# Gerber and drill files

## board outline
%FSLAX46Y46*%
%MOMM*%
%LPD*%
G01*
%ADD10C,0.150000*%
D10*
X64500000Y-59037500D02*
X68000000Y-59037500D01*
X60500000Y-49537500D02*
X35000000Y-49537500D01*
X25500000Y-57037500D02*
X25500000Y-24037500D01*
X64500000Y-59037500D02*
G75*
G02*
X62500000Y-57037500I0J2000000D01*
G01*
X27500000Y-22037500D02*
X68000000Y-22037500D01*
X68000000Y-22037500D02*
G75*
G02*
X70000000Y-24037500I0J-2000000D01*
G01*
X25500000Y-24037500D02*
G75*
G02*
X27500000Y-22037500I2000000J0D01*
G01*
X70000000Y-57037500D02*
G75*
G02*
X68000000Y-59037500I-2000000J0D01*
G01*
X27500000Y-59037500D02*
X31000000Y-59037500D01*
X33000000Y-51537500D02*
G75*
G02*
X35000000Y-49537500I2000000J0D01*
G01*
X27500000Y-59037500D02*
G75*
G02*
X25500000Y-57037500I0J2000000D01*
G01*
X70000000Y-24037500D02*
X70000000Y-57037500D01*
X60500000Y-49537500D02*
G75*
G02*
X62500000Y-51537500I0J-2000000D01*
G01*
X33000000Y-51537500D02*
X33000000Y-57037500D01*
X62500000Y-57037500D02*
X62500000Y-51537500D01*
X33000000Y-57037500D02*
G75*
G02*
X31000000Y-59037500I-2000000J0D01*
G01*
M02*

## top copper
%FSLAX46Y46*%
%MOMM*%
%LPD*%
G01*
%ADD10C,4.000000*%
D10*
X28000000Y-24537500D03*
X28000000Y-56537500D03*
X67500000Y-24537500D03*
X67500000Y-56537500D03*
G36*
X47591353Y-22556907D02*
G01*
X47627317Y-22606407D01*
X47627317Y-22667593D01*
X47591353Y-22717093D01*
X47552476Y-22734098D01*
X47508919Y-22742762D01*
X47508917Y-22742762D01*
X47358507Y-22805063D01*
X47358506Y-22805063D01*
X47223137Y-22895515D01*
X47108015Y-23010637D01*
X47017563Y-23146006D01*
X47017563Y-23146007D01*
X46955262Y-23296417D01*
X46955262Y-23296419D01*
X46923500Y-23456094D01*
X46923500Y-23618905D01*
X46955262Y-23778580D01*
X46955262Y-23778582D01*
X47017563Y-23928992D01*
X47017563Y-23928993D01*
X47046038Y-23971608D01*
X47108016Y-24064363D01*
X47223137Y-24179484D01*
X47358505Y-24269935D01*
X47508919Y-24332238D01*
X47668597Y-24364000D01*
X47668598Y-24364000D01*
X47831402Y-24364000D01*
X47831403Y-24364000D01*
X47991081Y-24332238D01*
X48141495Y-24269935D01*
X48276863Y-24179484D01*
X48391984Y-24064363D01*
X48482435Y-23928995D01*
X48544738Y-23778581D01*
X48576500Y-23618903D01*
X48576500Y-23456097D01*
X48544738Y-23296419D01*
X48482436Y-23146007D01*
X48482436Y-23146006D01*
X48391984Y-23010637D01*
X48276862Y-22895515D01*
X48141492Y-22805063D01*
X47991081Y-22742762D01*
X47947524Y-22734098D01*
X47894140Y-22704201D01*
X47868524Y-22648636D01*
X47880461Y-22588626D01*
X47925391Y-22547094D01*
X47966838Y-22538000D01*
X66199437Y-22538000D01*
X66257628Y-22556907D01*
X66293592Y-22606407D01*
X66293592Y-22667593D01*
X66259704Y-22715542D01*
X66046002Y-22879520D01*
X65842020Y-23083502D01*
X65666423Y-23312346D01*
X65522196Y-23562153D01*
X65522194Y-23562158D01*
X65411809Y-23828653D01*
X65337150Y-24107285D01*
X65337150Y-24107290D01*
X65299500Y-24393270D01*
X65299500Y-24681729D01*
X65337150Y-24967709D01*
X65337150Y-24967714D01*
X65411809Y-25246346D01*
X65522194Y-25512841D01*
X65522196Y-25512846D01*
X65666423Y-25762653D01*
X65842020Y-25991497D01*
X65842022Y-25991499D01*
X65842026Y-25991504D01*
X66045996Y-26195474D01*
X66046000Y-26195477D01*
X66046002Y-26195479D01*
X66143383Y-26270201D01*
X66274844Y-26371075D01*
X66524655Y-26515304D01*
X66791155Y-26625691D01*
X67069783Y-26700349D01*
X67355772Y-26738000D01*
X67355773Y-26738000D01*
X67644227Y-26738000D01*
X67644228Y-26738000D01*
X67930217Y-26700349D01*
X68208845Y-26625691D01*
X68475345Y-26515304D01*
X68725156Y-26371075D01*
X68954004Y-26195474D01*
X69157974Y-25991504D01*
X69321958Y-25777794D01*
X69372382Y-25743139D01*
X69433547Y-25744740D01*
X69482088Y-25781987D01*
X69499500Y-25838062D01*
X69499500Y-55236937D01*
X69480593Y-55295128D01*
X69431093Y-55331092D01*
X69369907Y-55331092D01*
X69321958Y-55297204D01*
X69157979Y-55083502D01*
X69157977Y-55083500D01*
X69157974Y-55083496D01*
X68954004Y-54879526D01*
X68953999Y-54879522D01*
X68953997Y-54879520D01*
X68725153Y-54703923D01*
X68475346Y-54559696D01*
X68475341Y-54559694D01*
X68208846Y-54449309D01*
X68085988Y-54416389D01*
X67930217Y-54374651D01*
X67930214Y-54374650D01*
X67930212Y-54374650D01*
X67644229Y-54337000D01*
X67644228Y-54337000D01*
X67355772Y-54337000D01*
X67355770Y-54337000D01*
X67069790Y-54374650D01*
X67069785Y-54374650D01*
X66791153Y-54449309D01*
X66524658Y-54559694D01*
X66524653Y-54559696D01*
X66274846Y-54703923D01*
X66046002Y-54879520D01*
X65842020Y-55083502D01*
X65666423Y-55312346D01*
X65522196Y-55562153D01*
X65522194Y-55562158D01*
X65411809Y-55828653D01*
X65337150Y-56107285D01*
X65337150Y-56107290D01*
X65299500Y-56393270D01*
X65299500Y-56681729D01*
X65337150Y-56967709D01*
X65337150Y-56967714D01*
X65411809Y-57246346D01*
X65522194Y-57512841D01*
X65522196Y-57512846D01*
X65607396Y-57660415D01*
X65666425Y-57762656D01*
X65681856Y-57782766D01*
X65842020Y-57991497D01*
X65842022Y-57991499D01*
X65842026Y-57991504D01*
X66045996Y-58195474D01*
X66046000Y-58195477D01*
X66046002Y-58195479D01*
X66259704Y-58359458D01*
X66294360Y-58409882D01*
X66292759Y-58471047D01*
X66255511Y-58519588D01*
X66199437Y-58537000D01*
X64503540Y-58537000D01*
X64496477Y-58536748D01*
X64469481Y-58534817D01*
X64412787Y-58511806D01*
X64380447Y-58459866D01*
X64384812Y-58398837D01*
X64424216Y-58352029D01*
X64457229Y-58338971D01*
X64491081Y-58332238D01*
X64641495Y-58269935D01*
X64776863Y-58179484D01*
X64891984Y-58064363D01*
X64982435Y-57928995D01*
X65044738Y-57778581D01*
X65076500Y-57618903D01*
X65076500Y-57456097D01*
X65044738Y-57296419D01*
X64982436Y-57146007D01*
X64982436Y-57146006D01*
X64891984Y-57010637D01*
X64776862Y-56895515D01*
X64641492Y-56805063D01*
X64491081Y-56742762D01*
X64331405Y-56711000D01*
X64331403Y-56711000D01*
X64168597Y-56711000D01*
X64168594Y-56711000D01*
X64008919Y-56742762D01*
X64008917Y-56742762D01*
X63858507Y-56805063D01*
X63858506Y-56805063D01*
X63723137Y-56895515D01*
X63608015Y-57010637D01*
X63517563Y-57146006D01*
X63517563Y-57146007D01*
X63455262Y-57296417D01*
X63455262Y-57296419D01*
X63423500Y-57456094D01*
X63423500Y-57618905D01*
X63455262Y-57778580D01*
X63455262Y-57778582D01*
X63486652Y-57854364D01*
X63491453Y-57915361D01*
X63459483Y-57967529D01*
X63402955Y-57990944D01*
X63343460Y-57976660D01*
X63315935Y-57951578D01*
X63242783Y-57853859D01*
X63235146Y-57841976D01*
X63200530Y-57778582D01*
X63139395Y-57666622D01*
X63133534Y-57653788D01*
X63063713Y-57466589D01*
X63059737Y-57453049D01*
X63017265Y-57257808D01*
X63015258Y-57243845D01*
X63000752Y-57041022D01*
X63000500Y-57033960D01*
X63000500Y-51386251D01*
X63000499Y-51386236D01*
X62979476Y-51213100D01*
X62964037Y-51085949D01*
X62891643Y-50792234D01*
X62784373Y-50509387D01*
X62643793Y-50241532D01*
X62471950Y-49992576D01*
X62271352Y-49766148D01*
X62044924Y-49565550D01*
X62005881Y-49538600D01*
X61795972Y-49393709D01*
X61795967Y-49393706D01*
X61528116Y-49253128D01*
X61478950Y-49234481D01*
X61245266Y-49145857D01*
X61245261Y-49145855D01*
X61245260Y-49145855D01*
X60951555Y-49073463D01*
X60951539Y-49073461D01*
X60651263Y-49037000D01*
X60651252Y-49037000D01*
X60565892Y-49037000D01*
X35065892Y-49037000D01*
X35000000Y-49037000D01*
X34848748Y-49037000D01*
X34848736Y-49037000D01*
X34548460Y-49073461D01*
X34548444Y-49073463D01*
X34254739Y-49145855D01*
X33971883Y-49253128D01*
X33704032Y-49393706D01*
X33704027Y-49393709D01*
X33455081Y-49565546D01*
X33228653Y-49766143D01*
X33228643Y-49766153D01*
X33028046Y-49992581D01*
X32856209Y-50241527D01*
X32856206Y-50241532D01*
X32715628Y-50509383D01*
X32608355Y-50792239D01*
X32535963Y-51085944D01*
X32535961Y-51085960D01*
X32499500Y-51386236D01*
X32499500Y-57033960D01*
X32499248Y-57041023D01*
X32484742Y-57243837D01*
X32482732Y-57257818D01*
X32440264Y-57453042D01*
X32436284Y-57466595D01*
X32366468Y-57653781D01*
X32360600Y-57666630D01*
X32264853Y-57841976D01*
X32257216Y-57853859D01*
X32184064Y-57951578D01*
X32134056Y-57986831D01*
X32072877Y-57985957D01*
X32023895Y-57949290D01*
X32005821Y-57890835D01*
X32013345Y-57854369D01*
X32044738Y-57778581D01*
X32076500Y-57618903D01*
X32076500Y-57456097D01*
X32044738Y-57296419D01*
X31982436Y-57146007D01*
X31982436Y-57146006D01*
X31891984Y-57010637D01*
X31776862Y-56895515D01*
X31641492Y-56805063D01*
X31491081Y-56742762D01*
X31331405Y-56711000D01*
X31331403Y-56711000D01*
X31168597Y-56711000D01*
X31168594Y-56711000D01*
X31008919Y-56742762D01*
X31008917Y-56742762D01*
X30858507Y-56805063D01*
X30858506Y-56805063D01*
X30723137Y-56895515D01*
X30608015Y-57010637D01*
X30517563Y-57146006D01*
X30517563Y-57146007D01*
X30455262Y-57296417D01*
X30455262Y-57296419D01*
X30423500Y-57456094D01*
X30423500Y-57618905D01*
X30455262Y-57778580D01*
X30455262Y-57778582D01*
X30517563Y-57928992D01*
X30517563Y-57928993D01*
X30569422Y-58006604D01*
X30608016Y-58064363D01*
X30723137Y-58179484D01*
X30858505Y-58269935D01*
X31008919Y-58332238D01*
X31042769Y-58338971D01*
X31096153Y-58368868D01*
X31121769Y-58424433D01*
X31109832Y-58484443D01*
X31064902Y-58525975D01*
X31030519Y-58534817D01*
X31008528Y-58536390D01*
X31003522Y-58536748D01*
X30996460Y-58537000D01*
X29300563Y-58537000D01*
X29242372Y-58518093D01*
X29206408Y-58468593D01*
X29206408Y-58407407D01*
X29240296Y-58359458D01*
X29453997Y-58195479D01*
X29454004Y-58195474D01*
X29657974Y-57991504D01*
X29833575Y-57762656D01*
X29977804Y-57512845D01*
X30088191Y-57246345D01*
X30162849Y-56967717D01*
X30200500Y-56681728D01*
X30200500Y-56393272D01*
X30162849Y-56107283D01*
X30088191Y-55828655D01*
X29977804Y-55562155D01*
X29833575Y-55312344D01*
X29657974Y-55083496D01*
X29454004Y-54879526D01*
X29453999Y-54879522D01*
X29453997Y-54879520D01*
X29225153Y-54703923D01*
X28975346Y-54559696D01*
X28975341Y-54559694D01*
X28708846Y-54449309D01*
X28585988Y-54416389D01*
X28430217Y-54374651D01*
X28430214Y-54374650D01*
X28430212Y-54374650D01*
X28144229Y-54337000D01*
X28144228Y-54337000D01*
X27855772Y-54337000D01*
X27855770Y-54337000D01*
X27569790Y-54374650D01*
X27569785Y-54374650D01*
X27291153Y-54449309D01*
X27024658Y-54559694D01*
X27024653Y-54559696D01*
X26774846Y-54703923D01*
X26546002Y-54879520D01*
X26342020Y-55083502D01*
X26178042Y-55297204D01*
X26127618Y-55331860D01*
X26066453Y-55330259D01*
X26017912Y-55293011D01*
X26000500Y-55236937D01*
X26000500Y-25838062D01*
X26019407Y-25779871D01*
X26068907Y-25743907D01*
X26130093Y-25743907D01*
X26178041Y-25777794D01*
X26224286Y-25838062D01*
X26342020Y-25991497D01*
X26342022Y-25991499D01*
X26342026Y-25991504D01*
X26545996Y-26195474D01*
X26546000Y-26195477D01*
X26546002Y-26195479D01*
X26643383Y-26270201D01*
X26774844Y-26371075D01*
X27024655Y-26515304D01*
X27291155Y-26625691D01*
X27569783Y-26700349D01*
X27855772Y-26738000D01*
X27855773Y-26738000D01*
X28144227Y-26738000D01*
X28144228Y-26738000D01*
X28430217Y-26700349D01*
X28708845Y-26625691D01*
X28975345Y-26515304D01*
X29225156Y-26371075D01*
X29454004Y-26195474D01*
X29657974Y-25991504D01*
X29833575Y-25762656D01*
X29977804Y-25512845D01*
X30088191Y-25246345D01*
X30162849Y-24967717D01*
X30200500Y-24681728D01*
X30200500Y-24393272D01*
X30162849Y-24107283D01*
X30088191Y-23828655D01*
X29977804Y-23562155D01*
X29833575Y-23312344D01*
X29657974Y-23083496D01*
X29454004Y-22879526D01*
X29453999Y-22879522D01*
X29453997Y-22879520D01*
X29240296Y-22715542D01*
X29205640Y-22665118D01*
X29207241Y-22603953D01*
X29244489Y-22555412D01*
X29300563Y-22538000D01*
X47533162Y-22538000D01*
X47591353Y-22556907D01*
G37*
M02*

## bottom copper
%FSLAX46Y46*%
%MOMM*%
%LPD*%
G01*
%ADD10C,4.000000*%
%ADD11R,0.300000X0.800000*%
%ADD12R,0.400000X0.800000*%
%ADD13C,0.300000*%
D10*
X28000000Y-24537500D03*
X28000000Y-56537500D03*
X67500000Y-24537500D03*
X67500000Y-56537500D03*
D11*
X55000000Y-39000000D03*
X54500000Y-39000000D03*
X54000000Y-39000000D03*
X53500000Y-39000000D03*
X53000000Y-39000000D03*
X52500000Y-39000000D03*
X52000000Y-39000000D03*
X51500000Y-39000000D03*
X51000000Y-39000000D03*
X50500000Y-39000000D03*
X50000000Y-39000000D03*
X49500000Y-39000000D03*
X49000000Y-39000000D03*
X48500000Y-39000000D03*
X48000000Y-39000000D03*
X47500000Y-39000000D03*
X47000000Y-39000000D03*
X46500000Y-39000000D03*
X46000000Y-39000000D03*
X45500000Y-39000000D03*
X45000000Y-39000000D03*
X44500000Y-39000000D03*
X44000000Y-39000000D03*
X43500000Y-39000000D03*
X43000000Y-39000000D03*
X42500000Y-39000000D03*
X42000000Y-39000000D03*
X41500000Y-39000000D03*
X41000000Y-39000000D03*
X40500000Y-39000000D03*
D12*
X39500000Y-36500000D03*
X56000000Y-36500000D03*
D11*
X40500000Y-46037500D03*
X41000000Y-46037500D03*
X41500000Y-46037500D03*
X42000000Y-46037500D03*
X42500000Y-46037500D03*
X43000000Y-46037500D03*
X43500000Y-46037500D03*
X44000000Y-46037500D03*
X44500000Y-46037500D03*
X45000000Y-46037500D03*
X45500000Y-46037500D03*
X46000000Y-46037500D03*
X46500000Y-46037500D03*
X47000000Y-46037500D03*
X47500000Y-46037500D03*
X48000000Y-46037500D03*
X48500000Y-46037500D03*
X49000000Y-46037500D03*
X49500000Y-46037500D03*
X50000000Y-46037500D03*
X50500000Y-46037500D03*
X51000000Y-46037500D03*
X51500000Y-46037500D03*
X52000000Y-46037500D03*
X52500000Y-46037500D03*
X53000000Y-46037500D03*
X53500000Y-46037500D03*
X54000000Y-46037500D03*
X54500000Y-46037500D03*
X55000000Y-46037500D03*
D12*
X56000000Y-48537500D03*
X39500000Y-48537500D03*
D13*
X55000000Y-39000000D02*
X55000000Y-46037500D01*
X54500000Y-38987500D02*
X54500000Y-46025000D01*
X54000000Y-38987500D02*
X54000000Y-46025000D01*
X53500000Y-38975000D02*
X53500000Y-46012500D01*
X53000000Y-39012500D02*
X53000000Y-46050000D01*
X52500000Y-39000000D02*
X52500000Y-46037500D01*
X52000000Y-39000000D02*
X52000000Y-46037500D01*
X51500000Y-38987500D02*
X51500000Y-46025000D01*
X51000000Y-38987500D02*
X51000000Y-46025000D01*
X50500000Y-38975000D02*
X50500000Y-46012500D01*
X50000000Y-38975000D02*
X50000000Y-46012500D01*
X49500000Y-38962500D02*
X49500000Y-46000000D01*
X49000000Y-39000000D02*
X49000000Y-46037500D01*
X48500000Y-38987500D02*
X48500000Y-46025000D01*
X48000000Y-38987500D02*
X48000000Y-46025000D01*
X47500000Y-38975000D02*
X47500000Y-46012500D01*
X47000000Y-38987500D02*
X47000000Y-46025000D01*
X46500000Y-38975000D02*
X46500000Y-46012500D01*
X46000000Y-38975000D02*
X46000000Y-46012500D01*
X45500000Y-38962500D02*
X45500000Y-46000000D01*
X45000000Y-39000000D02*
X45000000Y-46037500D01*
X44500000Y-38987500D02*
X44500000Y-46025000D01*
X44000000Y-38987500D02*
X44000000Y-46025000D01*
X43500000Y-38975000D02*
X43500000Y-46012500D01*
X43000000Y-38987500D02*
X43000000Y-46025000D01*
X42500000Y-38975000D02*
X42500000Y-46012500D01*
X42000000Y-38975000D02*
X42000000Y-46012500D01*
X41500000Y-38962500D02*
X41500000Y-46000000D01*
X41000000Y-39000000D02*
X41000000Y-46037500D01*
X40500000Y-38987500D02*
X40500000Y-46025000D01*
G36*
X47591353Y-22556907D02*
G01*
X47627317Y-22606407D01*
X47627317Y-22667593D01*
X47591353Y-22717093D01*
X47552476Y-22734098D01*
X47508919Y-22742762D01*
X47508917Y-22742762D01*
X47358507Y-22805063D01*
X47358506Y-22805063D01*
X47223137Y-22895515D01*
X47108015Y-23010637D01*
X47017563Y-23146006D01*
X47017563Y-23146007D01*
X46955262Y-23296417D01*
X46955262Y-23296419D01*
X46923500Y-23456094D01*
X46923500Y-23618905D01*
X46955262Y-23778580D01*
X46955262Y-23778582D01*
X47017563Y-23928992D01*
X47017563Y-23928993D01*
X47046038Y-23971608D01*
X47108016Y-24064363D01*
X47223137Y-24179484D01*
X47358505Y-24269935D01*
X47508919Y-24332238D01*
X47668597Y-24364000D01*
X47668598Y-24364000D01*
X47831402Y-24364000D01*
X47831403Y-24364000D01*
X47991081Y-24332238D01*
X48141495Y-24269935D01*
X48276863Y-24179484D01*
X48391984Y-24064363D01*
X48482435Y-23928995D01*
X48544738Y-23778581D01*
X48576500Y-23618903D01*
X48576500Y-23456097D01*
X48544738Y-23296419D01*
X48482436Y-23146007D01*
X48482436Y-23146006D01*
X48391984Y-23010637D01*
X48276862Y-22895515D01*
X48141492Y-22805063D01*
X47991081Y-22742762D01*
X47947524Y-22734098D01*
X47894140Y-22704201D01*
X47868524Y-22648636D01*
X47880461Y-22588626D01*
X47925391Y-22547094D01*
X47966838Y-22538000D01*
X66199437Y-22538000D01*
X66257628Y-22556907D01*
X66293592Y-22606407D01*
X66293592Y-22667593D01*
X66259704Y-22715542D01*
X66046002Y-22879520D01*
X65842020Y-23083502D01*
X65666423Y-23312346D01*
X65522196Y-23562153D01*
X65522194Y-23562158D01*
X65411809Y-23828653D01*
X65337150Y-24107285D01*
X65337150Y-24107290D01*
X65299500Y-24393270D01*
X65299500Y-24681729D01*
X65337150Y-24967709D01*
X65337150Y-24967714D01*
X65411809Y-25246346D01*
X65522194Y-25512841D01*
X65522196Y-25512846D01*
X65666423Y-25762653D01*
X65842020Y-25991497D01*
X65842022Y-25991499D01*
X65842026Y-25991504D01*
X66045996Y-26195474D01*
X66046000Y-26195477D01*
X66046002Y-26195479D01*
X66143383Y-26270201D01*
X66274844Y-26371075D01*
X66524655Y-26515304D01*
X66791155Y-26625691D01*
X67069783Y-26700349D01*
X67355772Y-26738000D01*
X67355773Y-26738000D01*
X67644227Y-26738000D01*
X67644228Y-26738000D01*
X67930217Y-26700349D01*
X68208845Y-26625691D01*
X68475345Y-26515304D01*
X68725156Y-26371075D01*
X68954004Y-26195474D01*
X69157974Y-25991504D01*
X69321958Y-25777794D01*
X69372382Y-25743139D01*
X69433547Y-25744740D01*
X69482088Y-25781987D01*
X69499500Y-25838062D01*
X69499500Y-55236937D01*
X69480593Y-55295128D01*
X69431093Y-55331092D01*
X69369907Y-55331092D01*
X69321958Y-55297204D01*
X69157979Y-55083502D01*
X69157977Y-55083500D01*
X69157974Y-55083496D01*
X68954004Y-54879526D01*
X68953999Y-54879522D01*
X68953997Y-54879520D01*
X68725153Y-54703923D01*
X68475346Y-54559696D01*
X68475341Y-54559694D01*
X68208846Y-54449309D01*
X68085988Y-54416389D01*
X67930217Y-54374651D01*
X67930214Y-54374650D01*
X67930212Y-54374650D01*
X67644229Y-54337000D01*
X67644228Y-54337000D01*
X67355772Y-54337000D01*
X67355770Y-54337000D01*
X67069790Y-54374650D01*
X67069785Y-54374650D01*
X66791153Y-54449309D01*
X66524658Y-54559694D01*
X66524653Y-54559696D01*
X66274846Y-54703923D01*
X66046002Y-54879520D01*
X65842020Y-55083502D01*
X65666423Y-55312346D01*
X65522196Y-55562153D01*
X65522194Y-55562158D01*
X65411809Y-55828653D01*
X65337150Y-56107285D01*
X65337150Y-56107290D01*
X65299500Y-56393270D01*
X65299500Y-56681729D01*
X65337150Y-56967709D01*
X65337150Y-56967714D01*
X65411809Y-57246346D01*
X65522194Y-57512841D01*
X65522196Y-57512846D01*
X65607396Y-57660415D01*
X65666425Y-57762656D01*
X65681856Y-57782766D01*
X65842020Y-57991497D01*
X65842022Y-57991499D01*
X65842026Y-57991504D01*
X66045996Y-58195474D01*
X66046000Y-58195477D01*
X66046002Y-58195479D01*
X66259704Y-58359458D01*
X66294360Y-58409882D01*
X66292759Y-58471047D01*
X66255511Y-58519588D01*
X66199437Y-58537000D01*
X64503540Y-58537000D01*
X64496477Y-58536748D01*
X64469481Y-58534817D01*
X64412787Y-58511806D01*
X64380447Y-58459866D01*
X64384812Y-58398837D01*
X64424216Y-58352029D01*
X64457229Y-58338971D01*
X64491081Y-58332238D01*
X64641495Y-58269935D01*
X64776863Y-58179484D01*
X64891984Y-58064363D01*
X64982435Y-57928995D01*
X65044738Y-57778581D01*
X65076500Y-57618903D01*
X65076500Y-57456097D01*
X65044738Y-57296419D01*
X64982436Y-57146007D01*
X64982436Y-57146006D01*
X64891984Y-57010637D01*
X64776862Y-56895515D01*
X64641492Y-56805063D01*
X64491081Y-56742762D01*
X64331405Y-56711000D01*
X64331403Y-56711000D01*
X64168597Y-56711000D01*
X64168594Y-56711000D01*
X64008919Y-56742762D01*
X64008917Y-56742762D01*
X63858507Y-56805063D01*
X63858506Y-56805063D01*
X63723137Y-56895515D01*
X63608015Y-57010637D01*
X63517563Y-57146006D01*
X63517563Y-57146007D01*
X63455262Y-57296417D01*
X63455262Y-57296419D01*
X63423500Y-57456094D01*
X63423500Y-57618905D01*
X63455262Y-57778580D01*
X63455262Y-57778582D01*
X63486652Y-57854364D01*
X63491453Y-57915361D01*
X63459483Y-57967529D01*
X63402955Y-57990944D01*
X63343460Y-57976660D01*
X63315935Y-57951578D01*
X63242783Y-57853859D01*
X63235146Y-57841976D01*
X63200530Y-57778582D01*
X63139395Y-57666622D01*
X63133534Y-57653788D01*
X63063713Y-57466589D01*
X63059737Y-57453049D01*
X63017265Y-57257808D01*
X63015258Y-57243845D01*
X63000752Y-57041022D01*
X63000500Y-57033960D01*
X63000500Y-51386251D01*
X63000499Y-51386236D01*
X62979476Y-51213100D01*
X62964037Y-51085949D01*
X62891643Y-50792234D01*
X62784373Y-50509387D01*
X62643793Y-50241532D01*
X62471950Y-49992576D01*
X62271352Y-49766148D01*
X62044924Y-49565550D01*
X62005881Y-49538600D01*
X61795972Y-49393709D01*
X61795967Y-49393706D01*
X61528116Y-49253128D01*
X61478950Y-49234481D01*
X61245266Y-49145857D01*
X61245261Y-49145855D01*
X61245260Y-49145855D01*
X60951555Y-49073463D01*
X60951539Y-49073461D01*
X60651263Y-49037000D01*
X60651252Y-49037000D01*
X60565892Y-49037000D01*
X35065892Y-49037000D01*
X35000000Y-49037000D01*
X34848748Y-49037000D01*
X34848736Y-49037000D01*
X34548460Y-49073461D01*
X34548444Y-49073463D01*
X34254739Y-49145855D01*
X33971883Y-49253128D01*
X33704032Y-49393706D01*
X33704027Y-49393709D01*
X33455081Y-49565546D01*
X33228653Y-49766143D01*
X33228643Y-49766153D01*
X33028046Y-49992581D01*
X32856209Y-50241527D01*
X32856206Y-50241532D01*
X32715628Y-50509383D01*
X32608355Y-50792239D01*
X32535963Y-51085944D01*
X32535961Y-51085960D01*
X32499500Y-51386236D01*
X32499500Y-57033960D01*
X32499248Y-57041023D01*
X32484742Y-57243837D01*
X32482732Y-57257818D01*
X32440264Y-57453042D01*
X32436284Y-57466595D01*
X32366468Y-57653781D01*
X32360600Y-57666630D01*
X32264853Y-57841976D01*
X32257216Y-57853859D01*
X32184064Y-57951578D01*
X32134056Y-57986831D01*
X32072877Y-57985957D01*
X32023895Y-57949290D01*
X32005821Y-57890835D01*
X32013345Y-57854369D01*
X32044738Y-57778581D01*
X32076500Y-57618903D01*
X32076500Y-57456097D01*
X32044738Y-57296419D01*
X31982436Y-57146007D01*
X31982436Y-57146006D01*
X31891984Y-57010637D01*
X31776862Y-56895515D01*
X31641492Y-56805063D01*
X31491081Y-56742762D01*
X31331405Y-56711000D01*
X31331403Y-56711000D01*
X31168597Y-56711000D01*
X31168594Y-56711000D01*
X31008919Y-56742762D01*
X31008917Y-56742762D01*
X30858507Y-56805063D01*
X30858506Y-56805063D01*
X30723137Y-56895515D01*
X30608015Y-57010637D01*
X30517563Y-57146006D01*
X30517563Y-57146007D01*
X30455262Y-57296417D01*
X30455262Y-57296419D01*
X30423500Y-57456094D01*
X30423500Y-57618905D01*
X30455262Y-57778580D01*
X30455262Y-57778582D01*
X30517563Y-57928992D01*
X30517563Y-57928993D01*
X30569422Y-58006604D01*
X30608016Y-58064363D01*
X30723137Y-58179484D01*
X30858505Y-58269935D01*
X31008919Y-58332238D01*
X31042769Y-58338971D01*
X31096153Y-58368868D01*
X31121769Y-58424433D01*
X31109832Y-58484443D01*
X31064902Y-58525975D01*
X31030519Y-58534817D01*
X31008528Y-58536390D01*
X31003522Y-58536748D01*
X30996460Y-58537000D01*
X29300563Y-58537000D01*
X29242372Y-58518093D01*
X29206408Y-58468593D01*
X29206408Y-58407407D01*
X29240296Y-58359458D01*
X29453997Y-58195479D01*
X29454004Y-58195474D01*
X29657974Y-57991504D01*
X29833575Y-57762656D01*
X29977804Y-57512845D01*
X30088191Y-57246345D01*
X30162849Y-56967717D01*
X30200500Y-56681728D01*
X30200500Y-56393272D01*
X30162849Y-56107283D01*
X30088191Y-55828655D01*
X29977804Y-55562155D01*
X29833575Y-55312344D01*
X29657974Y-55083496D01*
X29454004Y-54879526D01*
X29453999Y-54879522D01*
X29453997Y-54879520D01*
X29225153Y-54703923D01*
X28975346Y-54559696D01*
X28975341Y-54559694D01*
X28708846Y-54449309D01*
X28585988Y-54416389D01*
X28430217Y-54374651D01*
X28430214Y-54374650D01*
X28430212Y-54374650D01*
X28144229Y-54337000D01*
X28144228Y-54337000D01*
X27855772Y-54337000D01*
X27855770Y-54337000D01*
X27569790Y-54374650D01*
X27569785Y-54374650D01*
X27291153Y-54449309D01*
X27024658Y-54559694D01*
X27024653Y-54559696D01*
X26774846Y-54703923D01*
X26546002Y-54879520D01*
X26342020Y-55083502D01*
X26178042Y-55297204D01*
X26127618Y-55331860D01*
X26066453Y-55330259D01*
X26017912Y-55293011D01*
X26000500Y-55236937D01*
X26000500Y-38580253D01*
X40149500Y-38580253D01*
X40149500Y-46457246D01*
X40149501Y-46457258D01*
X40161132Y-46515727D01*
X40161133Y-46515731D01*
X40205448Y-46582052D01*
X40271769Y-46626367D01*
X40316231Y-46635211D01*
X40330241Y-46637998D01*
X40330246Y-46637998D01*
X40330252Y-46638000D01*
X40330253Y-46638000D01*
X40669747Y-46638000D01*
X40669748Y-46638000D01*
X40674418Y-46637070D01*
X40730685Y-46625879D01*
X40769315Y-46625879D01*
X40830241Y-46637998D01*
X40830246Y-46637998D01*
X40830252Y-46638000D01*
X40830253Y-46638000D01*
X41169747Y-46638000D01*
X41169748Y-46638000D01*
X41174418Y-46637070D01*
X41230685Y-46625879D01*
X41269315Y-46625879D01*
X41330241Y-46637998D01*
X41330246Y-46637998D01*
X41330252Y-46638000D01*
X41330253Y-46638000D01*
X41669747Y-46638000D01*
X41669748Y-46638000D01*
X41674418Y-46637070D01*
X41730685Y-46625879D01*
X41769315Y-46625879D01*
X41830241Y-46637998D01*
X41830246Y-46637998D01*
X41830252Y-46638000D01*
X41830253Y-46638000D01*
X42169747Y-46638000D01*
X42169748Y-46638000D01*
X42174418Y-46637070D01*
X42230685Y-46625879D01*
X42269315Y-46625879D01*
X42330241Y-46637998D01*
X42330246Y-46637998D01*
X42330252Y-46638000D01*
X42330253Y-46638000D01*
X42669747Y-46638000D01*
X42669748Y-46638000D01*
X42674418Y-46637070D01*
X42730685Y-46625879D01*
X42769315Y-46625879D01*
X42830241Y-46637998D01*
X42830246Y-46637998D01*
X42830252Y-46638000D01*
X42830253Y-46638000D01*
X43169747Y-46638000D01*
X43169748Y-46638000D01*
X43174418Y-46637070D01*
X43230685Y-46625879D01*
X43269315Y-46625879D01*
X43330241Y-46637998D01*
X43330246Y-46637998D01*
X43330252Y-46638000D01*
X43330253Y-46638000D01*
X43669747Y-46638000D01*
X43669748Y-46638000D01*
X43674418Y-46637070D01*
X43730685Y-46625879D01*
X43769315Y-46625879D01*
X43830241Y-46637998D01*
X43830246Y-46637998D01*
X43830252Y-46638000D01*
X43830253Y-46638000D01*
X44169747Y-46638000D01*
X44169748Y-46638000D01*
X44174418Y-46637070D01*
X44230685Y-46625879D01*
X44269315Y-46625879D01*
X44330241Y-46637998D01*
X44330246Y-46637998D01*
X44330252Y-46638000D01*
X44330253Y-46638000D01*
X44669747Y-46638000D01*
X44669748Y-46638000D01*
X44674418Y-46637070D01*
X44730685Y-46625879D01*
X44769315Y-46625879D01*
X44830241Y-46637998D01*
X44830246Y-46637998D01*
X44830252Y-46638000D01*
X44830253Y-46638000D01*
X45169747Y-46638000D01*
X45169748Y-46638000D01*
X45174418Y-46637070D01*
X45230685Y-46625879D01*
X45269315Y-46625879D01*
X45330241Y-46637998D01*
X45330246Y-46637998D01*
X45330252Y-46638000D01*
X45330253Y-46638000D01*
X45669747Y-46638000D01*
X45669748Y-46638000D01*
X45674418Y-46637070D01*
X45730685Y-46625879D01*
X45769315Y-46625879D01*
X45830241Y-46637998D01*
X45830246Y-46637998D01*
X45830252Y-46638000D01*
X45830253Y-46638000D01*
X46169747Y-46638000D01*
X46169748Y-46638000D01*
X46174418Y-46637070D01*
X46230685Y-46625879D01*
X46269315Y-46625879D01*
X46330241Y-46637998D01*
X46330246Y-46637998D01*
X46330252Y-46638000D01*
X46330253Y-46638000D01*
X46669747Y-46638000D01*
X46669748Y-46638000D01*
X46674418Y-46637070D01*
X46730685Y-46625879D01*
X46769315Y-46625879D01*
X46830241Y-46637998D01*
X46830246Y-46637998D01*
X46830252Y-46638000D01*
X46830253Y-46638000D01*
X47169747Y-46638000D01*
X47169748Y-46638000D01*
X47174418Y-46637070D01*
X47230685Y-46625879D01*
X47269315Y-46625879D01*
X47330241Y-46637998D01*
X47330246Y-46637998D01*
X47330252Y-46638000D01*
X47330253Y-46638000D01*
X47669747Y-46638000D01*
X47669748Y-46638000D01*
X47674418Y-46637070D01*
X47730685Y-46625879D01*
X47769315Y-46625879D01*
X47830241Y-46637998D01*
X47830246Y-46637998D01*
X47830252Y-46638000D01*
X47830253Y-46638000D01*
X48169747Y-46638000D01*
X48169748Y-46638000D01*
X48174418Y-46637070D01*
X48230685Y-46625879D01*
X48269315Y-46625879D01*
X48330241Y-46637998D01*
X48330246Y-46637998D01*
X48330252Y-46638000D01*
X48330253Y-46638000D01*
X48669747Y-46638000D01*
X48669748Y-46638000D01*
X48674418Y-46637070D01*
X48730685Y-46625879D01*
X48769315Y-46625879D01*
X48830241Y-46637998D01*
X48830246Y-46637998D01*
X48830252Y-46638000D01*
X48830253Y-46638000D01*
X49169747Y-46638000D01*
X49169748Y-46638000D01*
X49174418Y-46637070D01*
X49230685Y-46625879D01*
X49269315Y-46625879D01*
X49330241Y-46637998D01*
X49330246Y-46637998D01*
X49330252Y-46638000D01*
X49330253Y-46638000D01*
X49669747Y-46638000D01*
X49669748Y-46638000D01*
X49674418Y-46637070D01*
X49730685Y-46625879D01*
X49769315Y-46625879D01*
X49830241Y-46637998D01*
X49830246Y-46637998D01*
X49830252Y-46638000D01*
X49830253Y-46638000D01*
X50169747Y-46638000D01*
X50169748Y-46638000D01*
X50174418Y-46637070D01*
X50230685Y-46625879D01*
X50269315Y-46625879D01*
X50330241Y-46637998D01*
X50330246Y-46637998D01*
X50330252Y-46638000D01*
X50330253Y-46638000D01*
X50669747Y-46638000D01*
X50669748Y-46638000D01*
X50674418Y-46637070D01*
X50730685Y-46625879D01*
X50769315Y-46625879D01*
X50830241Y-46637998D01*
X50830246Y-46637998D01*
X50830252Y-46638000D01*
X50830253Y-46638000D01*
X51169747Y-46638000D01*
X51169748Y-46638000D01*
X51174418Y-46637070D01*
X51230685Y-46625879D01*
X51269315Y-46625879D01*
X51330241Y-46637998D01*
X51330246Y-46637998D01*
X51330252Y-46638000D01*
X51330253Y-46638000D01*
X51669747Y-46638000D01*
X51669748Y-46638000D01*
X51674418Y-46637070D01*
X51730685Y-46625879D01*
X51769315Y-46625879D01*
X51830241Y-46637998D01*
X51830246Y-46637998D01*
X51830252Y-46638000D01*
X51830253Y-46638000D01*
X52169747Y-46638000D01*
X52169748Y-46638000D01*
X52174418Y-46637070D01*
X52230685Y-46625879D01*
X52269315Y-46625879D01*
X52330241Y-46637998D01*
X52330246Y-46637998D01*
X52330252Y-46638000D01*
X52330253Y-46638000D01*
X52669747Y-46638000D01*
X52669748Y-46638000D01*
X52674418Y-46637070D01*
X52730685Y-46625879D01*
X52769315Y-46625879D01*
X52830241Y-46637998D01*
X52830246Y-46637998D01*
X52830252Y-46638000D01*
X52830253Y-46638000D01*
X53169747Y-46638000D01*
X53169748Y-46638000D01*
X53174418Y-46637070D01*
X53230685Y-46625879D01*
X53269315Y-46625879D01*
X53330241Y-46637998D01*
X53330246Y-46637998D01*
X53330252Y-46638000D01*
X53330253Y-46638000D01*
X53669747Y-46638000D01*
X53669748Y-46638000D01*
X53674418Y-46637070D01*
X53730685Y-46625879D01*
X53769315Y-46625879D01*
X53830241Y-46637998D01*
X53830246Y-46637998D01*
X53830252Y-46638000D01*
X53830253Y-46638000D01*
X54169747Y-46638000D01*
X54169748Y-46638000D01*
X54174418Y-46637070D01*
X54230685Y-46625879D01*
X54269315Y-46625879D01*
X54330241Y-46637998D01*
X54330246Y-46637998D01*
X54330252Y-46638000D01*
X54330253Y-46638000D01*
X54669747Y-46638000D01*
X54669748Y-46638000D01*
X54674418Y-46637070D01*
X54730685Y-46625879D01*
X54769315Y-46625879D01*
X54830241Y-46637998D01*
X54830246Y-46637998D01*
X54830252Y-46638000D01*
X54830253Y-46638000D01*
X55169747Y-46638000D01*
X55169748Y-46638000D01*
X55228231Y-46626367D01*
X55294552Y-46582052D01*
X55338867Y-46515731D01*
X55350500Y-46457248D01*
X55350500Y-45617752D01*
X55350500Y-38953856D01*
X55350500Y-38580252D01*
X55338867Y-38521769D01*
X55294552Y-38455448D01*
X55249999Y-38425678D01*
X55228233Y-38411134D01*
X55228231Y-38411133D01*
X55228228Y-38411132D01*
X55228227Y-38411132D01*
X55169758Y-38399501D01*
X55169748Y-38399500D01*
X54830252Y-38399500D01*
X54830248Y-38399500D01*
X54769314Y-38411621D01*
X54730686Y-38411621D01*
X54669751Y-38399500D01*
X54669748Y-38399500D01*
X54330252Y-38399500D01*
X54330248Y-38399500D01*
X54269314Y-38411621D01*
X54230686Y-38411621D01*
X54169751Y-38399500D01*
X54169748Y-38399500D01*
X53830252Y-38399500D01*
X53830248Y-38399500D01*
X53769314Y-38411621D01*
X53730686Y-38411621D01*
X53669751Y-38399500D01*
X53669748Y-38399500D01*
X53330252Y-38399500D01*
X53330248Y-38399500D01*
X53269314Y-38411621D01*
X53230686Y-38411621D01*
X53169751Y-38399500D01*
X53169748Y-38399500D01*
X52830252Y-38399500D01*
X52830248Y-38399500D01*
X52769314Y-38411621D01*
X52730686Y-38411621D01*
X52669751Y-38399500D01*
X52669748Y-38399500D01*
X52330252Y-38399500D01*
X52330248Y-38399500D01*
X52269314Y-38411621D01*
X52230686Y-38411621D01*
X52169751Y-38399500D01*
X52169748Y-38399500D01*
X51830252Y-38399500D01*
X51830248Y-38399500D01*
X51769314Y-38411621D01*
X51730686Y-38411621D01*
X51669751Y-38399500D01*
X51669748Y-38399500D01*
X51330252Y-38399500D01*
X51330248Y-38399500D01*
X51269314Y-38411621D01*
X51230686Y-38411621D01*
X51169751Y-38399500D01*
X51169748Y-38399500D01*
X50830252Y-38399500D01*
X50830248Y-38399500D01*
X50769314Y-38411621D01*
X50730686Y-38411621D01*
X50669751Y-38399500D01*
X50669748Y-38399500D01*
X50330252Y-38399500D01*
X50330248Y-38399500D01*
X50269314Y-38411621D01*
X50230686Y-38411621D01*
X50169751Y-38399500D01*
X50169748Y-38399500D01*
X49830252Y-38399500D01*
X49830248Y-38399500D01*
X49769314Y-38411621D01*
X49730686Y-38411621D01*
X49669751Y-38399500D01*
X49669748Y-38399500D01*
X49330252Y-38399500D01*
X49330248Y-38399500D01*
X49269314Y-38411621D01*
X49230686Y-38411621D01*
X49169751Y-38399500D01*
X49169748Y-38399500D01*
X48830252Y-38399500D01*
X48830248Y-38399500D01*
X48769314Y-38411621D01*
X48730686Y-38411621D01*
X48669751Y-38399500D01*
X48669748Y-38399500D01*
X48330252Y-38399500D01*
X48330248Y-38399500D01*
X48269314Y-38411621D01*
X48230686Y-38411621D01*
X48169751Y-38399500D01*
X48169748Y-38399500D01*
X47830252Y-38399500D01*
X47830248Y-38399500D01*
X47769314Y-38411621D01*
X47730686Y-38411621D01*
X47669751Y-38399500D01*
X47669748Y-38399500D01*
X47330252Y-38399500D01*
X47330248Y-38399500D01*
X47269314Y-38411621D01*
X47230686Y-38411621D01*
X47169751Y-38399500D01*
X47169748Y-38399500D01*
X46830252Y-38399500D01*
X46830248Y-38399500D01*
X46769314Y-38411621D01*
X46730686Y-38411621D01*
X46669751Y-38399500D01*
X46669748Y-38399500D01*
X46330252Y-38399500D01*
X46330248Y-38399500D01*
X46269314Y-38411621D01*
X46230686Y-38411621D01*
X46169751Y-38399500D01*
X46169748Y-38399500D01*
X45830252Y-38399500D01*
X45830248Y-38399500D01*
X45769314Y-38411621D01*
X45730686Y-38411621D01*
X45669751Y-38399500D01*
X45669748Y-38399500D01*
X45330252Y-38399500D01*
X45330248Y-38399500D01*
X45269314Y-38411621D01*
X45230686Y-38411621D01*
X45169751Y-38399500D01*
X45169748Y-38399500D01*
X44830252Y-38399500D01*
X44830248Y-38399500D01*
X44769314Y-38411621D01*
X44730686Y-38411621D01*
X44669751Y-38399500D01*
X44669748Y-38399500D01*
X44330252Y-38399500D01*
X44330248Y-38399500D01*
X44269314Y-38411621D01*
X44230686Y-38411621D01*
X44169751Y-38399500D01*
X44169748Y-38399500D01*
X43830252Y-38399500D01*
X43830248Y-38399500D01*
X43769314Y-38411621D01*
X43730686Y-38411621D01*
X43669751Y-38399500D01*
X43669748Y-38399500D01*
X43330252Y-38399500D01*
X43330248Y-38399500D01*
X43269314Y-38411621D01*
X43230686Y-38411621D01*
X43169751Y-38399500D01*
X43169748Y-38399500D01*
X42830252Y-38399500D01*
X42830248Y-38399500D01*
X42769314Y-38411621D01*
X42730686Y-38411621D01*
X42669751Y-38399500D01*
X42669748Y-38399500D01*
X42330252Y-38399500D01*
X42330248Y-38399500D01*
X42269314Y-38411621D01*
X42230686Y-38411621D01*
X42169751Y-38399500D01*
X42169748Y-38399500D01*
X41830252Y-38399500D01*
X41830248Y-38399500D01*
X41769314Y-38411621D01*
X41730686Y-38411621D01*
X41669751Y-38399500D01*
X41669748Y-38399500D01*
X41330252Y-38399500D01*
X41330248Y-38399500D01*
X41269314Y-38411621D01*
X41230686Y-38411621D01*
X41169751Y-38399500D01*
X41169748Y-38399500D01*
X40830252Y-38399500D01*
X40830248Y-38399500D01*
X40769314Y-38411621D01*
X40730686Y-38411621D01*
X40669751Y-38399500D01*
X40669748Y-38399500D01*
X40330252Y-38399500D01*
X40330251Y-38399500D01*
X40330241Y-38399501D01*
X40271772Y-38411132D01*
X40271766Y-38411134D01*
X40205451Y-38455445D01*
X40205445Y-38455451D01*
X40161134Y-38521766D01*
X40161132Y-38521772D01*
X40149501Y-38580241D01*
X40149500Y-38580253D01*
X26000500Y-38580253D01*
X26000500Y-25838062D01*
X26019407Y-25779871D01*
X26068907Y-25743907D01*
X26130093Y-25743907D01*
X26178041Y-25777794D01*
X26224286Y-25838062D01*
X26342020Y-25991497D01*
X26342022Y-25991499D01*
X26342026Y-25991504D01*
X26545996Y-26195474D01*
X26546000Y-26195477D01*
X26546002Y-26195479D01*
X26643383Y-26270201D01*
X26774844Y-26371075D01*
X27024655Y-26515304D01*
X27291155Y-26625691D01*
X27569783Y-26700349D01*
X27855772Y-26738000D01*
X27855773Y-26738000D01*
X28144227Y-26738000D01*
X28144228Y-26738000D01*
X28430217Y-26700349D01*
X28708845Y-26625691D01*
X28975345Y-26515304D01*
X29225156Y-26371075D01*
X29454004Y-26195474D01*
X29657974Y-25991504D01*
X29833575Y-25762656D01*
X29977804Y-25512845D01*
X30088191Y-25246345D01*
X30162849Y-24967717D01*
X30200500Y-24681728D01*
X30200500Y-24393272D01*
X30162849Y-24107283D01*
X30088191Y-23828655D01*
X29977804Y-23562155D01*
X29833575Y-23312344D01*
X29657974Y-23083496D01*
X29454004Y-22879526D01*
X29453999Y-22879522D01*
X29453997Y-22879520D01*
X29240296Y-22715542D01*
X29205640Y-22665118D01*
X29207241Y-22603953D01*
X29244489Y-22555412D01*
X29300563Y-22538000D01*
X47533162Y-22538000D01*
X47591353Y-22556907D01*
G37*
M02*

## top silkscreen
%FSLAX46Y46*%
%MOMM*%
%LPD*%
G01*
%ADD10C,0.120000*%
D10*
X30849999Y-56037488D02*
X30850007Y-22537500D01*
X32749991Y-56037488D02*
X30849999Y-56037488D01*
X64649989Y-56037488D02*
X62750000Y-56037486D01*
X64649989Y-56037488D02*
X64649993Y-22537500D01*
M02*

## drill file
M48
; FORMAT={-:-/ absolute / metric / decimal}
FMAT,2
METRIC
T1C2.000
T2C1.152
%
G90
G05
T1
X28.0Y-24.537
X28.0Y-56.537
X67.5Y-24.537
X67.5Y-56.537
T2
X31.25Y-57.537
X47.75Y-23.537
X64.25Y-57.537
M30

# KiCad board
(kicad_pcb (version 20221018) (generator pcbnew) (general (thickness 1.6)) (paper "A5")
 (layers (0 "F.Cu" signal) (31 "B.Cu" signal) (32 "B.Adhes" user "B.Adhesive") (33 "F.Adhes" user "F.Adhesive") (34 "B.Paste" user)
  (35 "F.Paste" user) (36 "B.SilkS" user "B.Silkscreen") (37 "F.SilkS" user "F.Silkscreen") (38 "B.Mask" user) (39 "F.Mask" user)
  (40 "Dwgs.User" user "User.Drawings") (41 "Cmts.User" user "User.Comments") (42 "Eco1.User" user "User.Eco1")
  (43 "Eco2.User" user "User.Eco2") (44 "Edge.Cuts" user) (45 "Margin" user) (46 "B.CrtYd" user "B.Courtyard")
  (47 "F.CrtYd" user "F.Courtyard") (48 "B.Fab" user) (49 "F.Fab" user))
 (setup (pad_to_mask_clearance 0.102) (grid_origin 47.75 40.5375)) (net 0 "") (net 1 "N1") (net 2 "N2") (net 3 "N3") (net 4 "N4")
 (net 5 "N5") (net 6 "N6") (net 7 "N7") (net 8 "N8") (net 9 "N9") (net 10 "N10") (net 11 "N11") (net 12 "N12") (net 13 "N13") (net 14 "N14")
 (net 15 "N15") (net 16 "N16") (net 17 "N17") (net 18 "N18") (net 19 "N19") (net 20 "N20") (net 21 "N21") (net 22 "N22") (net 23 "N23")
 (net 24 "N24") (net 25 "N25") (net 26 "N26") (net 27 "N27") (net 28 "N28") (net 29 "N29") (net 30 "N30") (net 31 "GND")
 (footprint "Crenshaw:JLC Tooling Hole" (layer "F.Cu") (at 47.75 23.5375)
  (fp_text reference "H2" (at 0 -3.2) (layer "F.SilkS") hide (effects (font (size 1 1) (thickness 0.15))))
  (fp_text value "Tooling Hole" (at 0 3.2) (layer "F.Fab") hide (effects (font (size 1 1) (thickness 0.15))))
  (pad "" np_thru_hole circle (at 0 0) (size 1.152 1.152) (drill 1.152) (layers "F&B.Cu" "*.Mask") (clearance 0.074)))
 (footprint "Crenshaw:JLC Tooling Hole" (layer "F.Cu") (at 31.25 57.5375)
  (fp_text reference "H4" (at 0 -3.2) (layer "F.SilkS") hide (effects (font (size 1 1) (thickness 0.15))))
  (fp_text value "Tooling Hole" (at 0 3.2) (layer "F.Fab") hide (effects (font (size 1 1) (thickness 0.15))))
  (pad "" np_thru_hole circle (at 0 0) (size 1.152 1.152) (drill 1.152) (layers "F&B.Cu" "*.Mask") (clearance 0.074)))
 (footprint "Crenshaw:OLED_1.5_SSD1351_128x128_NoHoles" (layer "F.Cu") (at 47.75 40.5375)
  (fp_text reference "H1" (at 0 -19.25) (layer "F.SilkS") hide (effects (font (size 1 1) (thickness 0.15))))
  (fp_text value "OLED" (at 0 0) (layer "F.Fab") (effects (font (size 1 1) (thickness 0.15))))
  (pad "MP" thru_hole circle (at -19.75 -16) (size 4 4) (drill 2) (layers "*.Cu" "*.Mask"))
  (pad "MP" thru_hole circle (at -19.75 16) (size 4 4) (drill 2) (layers "*.Cu" "*.Mask"))
  (pad "MP" thru_hole circle (at 19.75 -16) (size 4 4) (drill 2) (layers "*.Cu" "*.Mask"))
  (pad "MP" thru_hole circle (at 19.75 16) (size 4 4) (drill 2) (layers "*.Cu" "*.Mask")))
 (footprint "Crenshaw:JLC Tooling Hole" (layer "F.Cu") (at 64.25 57.5375)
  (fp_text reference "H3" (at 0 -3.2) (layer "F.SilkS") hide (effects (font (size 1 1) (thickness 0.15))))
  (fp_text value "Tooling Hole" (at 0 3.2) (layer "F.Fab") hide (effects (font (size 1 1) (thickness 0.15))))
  (pad "" np_thru_hole circle (at 0 0) (size 1.152 1.152) (drill 1.152) (layers "F&B.Cu" "*.Mask") (clearance 0.074)))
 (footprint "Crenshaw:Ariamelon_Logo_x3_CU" (layer "B.Cu") (at 47.75 27.7375 180)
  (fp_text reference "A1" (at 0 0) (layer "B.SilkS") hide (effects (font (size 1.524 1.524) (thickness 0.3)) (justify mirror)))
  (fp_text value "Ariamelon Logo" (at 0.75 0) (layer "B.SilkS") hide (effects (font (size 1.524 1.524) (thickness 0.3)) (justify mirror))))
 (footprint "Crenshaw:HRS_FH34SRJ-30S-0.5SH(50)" (layer "B.Cu") (at 47.75 36.5)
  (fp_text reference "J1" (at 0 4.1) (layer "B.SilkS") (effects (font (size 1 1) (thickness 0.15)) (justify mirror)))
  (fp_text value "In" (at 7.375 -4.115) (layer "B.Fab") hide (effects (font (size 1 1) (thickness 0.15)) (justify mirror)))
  (pad "1" smd rect (at 7.25 2.5) (size 0.3 0.8) (layers "B.Cu" "B.Mask") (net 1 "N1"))
  (pad "2" smd rect (at 6.75 2.5) (size 0.3 0.8) (layers "B.Cu" "B.Mask") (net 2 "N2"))
  (pad "3" smd rect (at 6.25 2.5) (size 0.3 0.8) (layers "B.Cu" "B.Mask") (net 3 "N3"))
  (pad "4" smd rect (at 5.75 2.5) (size 0.3 0.8) (layers "B.Cu" "B.Mask") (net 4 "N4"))
  (pad "5" smd rect (at 5.25 2.5) (size 0.3 0.8) (layers "B.Cu" "B.Mask") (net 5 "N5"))
  (pad "6" smd rect (at 4.75 2.5) (size 0.3 0.8) (layers "B.Cu" "B.Mask") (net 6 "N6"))
  (pad "7" smd rect (at 4.25 2.5) (size 0.3 0.8) (layers "B.Cu" "B.Mask") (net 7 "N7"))
  (pad "8" smd rect (at 3.75 2.5) (size 0.3 0.8) (layers "B.Cu" "B.Mask") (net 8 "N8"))
  (pad "9" smd rect (at 3.25 2.5) (size 0.3 0.8) (layers "B.Cu" "B.Mask") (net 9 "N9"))
  (pad "10" smd rect (at 2.75 2.5) (size 0.3 0.8) (layers "B.Cu" "B.Mask") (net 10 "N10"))
  (pad "11" smd rect (at 2.25 2.5) (size 0.3 0.8) (layers "B.Cu" "B.Mask") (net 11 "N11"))
  (pad "12" smd rect (at 1.75 2.5) (size 0.3 0.8) (layers "B.Cu" "B.Mask") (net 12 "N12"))
  (pad "13" smd rect (at 1.25 2.5) (size 0.3 0.8) (layers "B.Cu" "B.Mask") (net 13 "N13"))
  (pad "14" smd rect (at 0.75 2.5) (size 0.3 0.8) (layers "B.Cu" "B.Mask") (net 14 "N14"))
  (pad "15" smd rect (at 0.25 2.5) (size 0.3 0.8) (layers "B.Cu" "B.Mask") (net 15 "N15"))
  (pad "16" smd rect (at -0.25 2.5) (size 0.3 0.8) (layers "B.Cu" "B.Mask") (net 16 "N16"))
  (pad "17" smd rect (at -0.75 2.5) (size 0.3 0.8) (layers "B.Cu" "B.Mask") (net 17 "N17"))
  (pad "18" smd rect (at -1.25 2.5) (size 0.3 0.8) (layers "B.Cu" "B.Mask") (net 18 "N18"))
  (pad "19" smd rect (at -1.75 2.5) (size 0.3 0.8) (layers "B.Cu" "B.Mask") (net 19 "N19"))
  (pad "20" smd rect (at -2.25 2.5) (size 0.3 0.8) (layers "B.Cu" "B.Mask") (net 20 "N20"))
  (pad "21" smd rect (at -2.75 2.5) (size 0.3 0.8) (layers "B.Cu" "B.Mask") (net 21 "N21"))
  (pad "22" smd rect (at -3.25 2.5) (size 0.3 0.8) (layers "B.Cu" "B.Mask") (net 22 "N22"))
  (pad "23" smd rect (at -3.75 2.5) (size 0.3 0.8) (layers "B.Cu" "B.Mask") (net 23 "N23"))
  (pad "24" smd rect (at -4.25 2.5) (size 0.3 0.8) (layers "B.Cu" "B.Mask") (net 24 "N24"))
  (pad "25" smd rect (at -4.75 2.5) (size 0.3 0.8) (layers "B.Cu" "B.Mask") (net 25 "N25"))
  (pad "26" smd rect (at -5.25 2.5) (size 0.3 0.8) (layers "B.Cu" "B.Mask") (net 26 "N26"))
  (pad "27" smd rect (at -5.75 2.5) (size 0.3 0.8) (layers "B.Cu" "B.Mask") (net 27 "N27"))
  (pad "28" smd rect (at -6.25 2.5) (size 0.3 0.8) (layers "B.Cu" "B.Mask") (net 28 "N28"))
  (pad "29" smd rect (at -6.75 2.5) (size 0.3 0.8) (layers "B.Cu" "B.Mask") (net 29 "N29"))
  (pad "30" smd rect (at -7.25 2.5) (size 0.3 0.8) (layers "B.Cu" "B.Mask") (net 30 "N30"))
  (pad "MP" smd rect (at -8.25 0) (size 0.4 0.8) (layers "B.Cu" "B.Paste" "B.Mask") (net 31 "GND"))
  (pad "MP" smd rect (at 8.25 0) (size 0.4 0.8) (layers "B.Cu" "B.Paste" "B.Mask") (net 31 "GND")))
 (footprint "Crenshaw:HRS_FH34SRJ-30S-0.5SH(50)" (layer "B.Cu") (at 47.75 48.5375 180)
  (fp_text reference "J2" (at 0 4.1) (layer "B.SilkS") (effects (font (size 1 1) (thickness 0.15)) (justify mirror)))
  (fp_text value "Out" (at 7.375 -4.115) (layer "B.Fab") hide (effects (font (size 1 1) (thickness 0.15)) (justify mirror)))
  (pad "1" smd rect (at 7.25 2.5 180) (size 0.3 0.8) (layers "B.Cu" "B.Mask") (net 30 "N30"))
  (pad "2" smd rect (at 6.75 2.5 180) (size 0.3 0.8) (layers "B.Cu" "B.Mask") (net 29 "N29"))
  (pad "3" smd rect (at 6.25 2.5 180) (size 0.3 0.8) (layers "B.Cu" "B.Mask") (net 28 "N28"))
  (pad "4" smd rect (at 5.75 2.5 180) (size 0.3 0.8) (layers "B.Cu" "B.Mask") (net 27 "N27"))
  (pad "5" smd rect (at 5.25 2.5 180) (size 0.3 0.8) (layers "B.Cu" "B.Mask") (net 26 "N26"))
  (pad "6" smd rect (at 4.75 2.5 180) (size 0.3 0.8) (layers "B.Cu" "B.Mask") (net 25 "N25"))
  (pad "7" smd rect (at 4.25 2.5 180) (size 0.3 0.8) (layers "B.Cu" "B.Mask") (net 24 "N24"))
  (pad "8" smd rect (at 3.75 2.5 180) (size 0.3 0.8) (layers "B.Cu" "B.Mask") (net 23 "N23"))
  (pad "9" smd rect (at 3.25 2.5 180) (size 0.3 0.8) (layers "B.Cu" "B.Mask") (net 22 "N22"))
  (pad "10" smd rect (at 2.75 2.5 180) (size 0.3 0.8) (layers "B.Cu" "B.Mask") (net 21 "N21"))
  (pad "11" smd rect (at 2.25 2.5 180) (size 0.3 0.8) (layers "B.Cu" "B.Mask") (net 20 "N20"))
  (pad "12" smd rect (at 1.75 2.5 180) (size 0.3 0.8) (layers "B.Cu" "B.Mask") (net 19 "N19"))
  (pad "13" smd rect (at 1.25 2.5 180) (size 0.3 0.8) (layers "B.Cu" "B.Mask") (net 18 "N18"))
  (pad "14" smd rect (at 0.75 2.5 180) (size 0.3 0.8) (layers "B.Cu" "B.Mask") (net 17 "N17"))
  (pad "15" smd rect (at 0.25 2.5 180) (size 0.3 0.8) (layers "B.Cu" "B.Mask") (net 16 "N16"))
  (pad "16" smd rect (at -0.25 2.5 180) (size 0.3 0.8) (layers "B.Cu" "B.Mask") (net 15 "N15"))
  (pad "17" smd rect (at -0.75 2.5 180) (size 0.3 0.8) (layers "B.Cu" "B.Mask") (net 14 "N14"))
  (pad "18" smd rect (at -1.25 2.5 180) (size 0.3 0.8) (layers "B.Cu" "B.Mask") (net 13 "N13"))
  (pad "19" smd rect (at -1.75 2.5 180) (size 0.3 0.8) (layers "B.Cu" "B.Mask") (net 12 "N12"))
  (pad "20" smd rect (at -2.25 2.5 180) (size 0.3 0.8) (layers "B.Cu" "B.Mask") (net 11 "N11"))
  (pad "21" smd rect (at -2.75 2.5 180) (size 0.3 0.8) (layers "B.Cu" "B.Mask") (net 10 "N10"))
  (pad "22" smd rect (at -3.25 2.5 180) (size 0.3 0.8) (layers "B.Cu" "B.Mask") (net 9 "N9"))
  (pad "23" smd rect (at -3.75 2.5 180) (size 0.3 0.8) (layers "B.Cu" "B.Mask") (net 8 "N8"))
  (pad "24" smd rect (at -4.25 2.5 180) (size 0.3 0.8) (layers "B.Cu" "B.Mask") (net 7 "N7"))
  (pad "25" smd rect (at -4.75 2.5 180) (size 0.3 0.8) (layers "B.Cu" "B.Mask") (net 6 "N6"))
  (pad "26" smd rect (at -5.25 2.5 180) (size 0.3 0.8) (layers "B.Cu" "B.Mask") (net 5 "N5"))
  (pad "27" smd rect (at -5.75 2.5 180) (size 0.3 0.8) (layers "B.Cu" "B.Mask") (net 4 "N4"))
  (pad "28" smd rect (at -6.25 2.5 180) (size 0.3 0.8) (layers "B.Cu" "B.Mask") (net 3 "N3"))
  (pad "29" smd rect (at -6.75 2.5 180) (size 0.3 0.8) (layers "B.Cu" "B.Mask") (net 2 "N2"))
  (pad "30" smd rect (at -7.25 2.5 180) (size 0.3 0.8) (layers "B.Cu" "B.Mask") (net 1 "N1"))
  (pad "MP" smd rect (at -8.25 0 180) (size 0.4 0.8) (layers "B.Cu" "B.Paste" "B.Mask") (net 31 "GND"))
  (pad "MP" smd rect (at 8.25 0 180) (size 0.4 0.8) (layers "B.Cu" "B.Paste" "B.Mask") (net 31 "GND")))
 (gr_line (start 30.849999 56.037488) (end 30.850007 22.5375) (stroke (width 0.12) (type default)) (layer "F.SilkS"))
 (gr_line (start 32.749991 56.037488) (end 30.849999 56.037488) (stroke (width 0.12) (type default)) (layer "F.SilkS"))
 (gr_line (start 64.649989 56.037488) (end 62.75 56.037486) (stroke (width 0.12) (type default)) (layer "F.SilkS"))
 (gr_line (start 64.649989 56.037488) (end 64.649993 22.5375) (stroke (width 0.12) (type default)) (layer "F.SilkS"))
 (gr_line (start 64.5 59.0375) (end 68 59.0375) (stroke (width 0.15) (type default)) (layer "Edge.Cuts"))
 (gr_line (start 60.5 49.5375) (end 35 49.5375) (stroke (width 0.15) (type default)) (layer "Edge.Cuts"))
 (gr_line (start 25.5 57.0375) (end 25.5 24.0375) (stroke (width 0.15) (type default)) (layer "Edge.Cuts"))
 (gr_arc (start 64.5 59.0375) (mid 63.085786 58.451714) (end 62.5 57.0375) (stroke (width 0.15) (type default)) (layer "Edge.Cuts"))
 (gr_line (start 27.5 22.0375) (end 68 22.0375) (stroke (width 0.15) (type default)) (layer "Edge.Cuts"))
 (gr_arc (start 68 22.0375) (mid 69.414214 22.623286) (end 70 24.0375) (stroke (width 0.15) (type default)) (layer "Edge.Cuts"))
 (gr_arc (start 25.5 24.0375) (mid 26.085786 22.623286) (end 27.5 22.0375) (stroke (width 0.15) (type default)) (layer "Edge.Cuts"))
 (gr_arc (start 70 57.0375) (mid 69.414214 58.451714) (end 68 59.0375) (stroke (width 0.15) (type default)) (layer "Edge.Cuts"))
 (gr_line (start 27.5 59.0375) (end 31 59.0375) (stroke (width 0.15) (type default)) (layer "Edge.Cuts"))
 (gr_arc (start 33 51.5375) (mid 33.585786 50.123286) (end 35 49.5375) (stroke (width 0.15) (type default)) (layer "Edge.Cuts"))
 (gr_arc (start 27.5 59.0375) (mid 26.085786 58.451714) (end 25.5 57.0375) (stroke (width 0.15) (type default)) (layer "Edge.Cuts"))
 (gr_line (start 70 24.0375) (end 70 57.0375) (stroke (width 0.15) (type default)) (layer "Edge.Cuts"))
 (gr_arc (start 60.5 49.5375) (mid 61.914214 50.123286) (end 62.5 51.5375) (stroke (width 0.15) (type default)) (layer "Edge.Cuts"))
 (gr_line (start 33 51.5375) (end 33 57.0375) (stroke (width 0.15) (type default)) (layer "Edge.Cuts"))
 (gr_line (start 62.5 57.0375) (end 62.5 51.5375) (stroke (width 0.15) (type default)) (layer "Edge.Cuts"))
 (gr_arc (start 33 57.0375) (mid 32.414214 58.451714) (end 31 59.0375) (stroke (width 0.15) (type default)) (layer "Edge.Cuts"))
 (segment (start 55 39) (end 55 46.0375) (width 0.3) (layer "B.Cu") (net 1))
 (segment (start 54.5 38.9875) (end 54.5 46.025) (width 0.3) (layer "B.Cu") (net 2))
 (segment (start 54 38.9875) (end 54 46.025) (width 0.3) (layer "B.Cu") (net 3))
 (segment (start 53.5 38.975) (end 53.5 46.0125) (width 0.3) (layer "B.Cu") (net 4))
 (segment (start 53 39.0125) (end 53 46.05) (width 0.3) (layer "B.Cu") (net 5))
 (segment (start 52.5 39) (end 52.5 46.0375) (width 0.3) (layer "B.Cu") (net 6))
 (segment (start 52 39) (end 52 46.0375) (width 0.3) (layer "B.Cu") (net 7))
 (segment (start 51.5 38.9875) (end 51.5 46.025) (width 0.3) (layer "B.Cu") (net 8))
 (segment (start 51 38.9875) (end 51 46.025) (width 0.3) (layer "B.Cu") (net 9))
 (segment (start 50.5 38.975) (end 50.5 46.0125) (width 0.3) (layer "B.Cu") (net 10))
 (segment (start 50 38.975) (end 50 46.0125) (width 0.3) (layer "B.Cu") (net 11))
 (segment (start 49.5 38.9625) (end 49.5 46) (width 0.3) (layer "B.Cu") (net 12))
 (segment (start 49 39) (end 49 46.0375) (width 0.3) (layer "B.Cu") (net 13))
 (segment (start 48.5 38.9875) (end 48.5 46.025) (width 0.3) (layer "B.Cu") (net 14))
 (segment (start 48 38.9875) (end 48 46.025) (width 0.3) (layer "B.Cu") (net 15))
 (segment (start 47.5 38.975) (end 47.5 46.0125) (width 0.3) (layer "B.Cu") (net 16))
 (segment (start 47 38.9875) (end 47 46.025) (width 0.3) (layer "B.Cu") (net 17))
 (segment (start 46.5 38.975) (end 46.5 46.0125) (width 0.3) (layer "B.Cu") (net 18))
 (segment (start 46 38.975) (end 46 46.0125) (width 0.3) (layer "B.Cu") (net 19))
 (segment (start 45.5 38.9625) (end 45.5 46) (width 0.3) (layer "B.Cu") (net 20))
 (segment (start 45 39) (end 45 46.0375) (width 0.3) (layer "B.Cu") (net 21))
 (segment (start 44.5 38.9875) (end 44.5 46.025) (width 0.3) (layer "B.Cu") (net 22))
 (segment (start 44 38.9875) (end 44 46.025) (width 0.3) (layer "B.Cu") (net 23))
 (segment (start 43.5 38.975) (end 43.5 46.0125) (width 0.3) (layer "B.Cu") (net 24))
 (segment (start 43 38.9875) (end 43 46.025) (width 0.3) (layer "B.Cu") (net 25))
 (segment (start 42.5 38.975) (end 42.5 46.0125) (width 0.3) (layer "B.Cu") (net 26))
 (segment (start 42 38.975) (end 42 46.0125) (width 0.3) (layer "B.Cu") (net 27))
 (segment (start 41.5 38.9625) (end 41.5 46) (width 0.3) (layer "B.Cu") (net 28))
 (segment (start 41 39) (end 41 46.0375) (width 0.3) (layer "B.Cu") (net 29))
 (segment (start 40.5 38.9875) (end 40.5 46.025) (width 0.3) (layer "B.Cu") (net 30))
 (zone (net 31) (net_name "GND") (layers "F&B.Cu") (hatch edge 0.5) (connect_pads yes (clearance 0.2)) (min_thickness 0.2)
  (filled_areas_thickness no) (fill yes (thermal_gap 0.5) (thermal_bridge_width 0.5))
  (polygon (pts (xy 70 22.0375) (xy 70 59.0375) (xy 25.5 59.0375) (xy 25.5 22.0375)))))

